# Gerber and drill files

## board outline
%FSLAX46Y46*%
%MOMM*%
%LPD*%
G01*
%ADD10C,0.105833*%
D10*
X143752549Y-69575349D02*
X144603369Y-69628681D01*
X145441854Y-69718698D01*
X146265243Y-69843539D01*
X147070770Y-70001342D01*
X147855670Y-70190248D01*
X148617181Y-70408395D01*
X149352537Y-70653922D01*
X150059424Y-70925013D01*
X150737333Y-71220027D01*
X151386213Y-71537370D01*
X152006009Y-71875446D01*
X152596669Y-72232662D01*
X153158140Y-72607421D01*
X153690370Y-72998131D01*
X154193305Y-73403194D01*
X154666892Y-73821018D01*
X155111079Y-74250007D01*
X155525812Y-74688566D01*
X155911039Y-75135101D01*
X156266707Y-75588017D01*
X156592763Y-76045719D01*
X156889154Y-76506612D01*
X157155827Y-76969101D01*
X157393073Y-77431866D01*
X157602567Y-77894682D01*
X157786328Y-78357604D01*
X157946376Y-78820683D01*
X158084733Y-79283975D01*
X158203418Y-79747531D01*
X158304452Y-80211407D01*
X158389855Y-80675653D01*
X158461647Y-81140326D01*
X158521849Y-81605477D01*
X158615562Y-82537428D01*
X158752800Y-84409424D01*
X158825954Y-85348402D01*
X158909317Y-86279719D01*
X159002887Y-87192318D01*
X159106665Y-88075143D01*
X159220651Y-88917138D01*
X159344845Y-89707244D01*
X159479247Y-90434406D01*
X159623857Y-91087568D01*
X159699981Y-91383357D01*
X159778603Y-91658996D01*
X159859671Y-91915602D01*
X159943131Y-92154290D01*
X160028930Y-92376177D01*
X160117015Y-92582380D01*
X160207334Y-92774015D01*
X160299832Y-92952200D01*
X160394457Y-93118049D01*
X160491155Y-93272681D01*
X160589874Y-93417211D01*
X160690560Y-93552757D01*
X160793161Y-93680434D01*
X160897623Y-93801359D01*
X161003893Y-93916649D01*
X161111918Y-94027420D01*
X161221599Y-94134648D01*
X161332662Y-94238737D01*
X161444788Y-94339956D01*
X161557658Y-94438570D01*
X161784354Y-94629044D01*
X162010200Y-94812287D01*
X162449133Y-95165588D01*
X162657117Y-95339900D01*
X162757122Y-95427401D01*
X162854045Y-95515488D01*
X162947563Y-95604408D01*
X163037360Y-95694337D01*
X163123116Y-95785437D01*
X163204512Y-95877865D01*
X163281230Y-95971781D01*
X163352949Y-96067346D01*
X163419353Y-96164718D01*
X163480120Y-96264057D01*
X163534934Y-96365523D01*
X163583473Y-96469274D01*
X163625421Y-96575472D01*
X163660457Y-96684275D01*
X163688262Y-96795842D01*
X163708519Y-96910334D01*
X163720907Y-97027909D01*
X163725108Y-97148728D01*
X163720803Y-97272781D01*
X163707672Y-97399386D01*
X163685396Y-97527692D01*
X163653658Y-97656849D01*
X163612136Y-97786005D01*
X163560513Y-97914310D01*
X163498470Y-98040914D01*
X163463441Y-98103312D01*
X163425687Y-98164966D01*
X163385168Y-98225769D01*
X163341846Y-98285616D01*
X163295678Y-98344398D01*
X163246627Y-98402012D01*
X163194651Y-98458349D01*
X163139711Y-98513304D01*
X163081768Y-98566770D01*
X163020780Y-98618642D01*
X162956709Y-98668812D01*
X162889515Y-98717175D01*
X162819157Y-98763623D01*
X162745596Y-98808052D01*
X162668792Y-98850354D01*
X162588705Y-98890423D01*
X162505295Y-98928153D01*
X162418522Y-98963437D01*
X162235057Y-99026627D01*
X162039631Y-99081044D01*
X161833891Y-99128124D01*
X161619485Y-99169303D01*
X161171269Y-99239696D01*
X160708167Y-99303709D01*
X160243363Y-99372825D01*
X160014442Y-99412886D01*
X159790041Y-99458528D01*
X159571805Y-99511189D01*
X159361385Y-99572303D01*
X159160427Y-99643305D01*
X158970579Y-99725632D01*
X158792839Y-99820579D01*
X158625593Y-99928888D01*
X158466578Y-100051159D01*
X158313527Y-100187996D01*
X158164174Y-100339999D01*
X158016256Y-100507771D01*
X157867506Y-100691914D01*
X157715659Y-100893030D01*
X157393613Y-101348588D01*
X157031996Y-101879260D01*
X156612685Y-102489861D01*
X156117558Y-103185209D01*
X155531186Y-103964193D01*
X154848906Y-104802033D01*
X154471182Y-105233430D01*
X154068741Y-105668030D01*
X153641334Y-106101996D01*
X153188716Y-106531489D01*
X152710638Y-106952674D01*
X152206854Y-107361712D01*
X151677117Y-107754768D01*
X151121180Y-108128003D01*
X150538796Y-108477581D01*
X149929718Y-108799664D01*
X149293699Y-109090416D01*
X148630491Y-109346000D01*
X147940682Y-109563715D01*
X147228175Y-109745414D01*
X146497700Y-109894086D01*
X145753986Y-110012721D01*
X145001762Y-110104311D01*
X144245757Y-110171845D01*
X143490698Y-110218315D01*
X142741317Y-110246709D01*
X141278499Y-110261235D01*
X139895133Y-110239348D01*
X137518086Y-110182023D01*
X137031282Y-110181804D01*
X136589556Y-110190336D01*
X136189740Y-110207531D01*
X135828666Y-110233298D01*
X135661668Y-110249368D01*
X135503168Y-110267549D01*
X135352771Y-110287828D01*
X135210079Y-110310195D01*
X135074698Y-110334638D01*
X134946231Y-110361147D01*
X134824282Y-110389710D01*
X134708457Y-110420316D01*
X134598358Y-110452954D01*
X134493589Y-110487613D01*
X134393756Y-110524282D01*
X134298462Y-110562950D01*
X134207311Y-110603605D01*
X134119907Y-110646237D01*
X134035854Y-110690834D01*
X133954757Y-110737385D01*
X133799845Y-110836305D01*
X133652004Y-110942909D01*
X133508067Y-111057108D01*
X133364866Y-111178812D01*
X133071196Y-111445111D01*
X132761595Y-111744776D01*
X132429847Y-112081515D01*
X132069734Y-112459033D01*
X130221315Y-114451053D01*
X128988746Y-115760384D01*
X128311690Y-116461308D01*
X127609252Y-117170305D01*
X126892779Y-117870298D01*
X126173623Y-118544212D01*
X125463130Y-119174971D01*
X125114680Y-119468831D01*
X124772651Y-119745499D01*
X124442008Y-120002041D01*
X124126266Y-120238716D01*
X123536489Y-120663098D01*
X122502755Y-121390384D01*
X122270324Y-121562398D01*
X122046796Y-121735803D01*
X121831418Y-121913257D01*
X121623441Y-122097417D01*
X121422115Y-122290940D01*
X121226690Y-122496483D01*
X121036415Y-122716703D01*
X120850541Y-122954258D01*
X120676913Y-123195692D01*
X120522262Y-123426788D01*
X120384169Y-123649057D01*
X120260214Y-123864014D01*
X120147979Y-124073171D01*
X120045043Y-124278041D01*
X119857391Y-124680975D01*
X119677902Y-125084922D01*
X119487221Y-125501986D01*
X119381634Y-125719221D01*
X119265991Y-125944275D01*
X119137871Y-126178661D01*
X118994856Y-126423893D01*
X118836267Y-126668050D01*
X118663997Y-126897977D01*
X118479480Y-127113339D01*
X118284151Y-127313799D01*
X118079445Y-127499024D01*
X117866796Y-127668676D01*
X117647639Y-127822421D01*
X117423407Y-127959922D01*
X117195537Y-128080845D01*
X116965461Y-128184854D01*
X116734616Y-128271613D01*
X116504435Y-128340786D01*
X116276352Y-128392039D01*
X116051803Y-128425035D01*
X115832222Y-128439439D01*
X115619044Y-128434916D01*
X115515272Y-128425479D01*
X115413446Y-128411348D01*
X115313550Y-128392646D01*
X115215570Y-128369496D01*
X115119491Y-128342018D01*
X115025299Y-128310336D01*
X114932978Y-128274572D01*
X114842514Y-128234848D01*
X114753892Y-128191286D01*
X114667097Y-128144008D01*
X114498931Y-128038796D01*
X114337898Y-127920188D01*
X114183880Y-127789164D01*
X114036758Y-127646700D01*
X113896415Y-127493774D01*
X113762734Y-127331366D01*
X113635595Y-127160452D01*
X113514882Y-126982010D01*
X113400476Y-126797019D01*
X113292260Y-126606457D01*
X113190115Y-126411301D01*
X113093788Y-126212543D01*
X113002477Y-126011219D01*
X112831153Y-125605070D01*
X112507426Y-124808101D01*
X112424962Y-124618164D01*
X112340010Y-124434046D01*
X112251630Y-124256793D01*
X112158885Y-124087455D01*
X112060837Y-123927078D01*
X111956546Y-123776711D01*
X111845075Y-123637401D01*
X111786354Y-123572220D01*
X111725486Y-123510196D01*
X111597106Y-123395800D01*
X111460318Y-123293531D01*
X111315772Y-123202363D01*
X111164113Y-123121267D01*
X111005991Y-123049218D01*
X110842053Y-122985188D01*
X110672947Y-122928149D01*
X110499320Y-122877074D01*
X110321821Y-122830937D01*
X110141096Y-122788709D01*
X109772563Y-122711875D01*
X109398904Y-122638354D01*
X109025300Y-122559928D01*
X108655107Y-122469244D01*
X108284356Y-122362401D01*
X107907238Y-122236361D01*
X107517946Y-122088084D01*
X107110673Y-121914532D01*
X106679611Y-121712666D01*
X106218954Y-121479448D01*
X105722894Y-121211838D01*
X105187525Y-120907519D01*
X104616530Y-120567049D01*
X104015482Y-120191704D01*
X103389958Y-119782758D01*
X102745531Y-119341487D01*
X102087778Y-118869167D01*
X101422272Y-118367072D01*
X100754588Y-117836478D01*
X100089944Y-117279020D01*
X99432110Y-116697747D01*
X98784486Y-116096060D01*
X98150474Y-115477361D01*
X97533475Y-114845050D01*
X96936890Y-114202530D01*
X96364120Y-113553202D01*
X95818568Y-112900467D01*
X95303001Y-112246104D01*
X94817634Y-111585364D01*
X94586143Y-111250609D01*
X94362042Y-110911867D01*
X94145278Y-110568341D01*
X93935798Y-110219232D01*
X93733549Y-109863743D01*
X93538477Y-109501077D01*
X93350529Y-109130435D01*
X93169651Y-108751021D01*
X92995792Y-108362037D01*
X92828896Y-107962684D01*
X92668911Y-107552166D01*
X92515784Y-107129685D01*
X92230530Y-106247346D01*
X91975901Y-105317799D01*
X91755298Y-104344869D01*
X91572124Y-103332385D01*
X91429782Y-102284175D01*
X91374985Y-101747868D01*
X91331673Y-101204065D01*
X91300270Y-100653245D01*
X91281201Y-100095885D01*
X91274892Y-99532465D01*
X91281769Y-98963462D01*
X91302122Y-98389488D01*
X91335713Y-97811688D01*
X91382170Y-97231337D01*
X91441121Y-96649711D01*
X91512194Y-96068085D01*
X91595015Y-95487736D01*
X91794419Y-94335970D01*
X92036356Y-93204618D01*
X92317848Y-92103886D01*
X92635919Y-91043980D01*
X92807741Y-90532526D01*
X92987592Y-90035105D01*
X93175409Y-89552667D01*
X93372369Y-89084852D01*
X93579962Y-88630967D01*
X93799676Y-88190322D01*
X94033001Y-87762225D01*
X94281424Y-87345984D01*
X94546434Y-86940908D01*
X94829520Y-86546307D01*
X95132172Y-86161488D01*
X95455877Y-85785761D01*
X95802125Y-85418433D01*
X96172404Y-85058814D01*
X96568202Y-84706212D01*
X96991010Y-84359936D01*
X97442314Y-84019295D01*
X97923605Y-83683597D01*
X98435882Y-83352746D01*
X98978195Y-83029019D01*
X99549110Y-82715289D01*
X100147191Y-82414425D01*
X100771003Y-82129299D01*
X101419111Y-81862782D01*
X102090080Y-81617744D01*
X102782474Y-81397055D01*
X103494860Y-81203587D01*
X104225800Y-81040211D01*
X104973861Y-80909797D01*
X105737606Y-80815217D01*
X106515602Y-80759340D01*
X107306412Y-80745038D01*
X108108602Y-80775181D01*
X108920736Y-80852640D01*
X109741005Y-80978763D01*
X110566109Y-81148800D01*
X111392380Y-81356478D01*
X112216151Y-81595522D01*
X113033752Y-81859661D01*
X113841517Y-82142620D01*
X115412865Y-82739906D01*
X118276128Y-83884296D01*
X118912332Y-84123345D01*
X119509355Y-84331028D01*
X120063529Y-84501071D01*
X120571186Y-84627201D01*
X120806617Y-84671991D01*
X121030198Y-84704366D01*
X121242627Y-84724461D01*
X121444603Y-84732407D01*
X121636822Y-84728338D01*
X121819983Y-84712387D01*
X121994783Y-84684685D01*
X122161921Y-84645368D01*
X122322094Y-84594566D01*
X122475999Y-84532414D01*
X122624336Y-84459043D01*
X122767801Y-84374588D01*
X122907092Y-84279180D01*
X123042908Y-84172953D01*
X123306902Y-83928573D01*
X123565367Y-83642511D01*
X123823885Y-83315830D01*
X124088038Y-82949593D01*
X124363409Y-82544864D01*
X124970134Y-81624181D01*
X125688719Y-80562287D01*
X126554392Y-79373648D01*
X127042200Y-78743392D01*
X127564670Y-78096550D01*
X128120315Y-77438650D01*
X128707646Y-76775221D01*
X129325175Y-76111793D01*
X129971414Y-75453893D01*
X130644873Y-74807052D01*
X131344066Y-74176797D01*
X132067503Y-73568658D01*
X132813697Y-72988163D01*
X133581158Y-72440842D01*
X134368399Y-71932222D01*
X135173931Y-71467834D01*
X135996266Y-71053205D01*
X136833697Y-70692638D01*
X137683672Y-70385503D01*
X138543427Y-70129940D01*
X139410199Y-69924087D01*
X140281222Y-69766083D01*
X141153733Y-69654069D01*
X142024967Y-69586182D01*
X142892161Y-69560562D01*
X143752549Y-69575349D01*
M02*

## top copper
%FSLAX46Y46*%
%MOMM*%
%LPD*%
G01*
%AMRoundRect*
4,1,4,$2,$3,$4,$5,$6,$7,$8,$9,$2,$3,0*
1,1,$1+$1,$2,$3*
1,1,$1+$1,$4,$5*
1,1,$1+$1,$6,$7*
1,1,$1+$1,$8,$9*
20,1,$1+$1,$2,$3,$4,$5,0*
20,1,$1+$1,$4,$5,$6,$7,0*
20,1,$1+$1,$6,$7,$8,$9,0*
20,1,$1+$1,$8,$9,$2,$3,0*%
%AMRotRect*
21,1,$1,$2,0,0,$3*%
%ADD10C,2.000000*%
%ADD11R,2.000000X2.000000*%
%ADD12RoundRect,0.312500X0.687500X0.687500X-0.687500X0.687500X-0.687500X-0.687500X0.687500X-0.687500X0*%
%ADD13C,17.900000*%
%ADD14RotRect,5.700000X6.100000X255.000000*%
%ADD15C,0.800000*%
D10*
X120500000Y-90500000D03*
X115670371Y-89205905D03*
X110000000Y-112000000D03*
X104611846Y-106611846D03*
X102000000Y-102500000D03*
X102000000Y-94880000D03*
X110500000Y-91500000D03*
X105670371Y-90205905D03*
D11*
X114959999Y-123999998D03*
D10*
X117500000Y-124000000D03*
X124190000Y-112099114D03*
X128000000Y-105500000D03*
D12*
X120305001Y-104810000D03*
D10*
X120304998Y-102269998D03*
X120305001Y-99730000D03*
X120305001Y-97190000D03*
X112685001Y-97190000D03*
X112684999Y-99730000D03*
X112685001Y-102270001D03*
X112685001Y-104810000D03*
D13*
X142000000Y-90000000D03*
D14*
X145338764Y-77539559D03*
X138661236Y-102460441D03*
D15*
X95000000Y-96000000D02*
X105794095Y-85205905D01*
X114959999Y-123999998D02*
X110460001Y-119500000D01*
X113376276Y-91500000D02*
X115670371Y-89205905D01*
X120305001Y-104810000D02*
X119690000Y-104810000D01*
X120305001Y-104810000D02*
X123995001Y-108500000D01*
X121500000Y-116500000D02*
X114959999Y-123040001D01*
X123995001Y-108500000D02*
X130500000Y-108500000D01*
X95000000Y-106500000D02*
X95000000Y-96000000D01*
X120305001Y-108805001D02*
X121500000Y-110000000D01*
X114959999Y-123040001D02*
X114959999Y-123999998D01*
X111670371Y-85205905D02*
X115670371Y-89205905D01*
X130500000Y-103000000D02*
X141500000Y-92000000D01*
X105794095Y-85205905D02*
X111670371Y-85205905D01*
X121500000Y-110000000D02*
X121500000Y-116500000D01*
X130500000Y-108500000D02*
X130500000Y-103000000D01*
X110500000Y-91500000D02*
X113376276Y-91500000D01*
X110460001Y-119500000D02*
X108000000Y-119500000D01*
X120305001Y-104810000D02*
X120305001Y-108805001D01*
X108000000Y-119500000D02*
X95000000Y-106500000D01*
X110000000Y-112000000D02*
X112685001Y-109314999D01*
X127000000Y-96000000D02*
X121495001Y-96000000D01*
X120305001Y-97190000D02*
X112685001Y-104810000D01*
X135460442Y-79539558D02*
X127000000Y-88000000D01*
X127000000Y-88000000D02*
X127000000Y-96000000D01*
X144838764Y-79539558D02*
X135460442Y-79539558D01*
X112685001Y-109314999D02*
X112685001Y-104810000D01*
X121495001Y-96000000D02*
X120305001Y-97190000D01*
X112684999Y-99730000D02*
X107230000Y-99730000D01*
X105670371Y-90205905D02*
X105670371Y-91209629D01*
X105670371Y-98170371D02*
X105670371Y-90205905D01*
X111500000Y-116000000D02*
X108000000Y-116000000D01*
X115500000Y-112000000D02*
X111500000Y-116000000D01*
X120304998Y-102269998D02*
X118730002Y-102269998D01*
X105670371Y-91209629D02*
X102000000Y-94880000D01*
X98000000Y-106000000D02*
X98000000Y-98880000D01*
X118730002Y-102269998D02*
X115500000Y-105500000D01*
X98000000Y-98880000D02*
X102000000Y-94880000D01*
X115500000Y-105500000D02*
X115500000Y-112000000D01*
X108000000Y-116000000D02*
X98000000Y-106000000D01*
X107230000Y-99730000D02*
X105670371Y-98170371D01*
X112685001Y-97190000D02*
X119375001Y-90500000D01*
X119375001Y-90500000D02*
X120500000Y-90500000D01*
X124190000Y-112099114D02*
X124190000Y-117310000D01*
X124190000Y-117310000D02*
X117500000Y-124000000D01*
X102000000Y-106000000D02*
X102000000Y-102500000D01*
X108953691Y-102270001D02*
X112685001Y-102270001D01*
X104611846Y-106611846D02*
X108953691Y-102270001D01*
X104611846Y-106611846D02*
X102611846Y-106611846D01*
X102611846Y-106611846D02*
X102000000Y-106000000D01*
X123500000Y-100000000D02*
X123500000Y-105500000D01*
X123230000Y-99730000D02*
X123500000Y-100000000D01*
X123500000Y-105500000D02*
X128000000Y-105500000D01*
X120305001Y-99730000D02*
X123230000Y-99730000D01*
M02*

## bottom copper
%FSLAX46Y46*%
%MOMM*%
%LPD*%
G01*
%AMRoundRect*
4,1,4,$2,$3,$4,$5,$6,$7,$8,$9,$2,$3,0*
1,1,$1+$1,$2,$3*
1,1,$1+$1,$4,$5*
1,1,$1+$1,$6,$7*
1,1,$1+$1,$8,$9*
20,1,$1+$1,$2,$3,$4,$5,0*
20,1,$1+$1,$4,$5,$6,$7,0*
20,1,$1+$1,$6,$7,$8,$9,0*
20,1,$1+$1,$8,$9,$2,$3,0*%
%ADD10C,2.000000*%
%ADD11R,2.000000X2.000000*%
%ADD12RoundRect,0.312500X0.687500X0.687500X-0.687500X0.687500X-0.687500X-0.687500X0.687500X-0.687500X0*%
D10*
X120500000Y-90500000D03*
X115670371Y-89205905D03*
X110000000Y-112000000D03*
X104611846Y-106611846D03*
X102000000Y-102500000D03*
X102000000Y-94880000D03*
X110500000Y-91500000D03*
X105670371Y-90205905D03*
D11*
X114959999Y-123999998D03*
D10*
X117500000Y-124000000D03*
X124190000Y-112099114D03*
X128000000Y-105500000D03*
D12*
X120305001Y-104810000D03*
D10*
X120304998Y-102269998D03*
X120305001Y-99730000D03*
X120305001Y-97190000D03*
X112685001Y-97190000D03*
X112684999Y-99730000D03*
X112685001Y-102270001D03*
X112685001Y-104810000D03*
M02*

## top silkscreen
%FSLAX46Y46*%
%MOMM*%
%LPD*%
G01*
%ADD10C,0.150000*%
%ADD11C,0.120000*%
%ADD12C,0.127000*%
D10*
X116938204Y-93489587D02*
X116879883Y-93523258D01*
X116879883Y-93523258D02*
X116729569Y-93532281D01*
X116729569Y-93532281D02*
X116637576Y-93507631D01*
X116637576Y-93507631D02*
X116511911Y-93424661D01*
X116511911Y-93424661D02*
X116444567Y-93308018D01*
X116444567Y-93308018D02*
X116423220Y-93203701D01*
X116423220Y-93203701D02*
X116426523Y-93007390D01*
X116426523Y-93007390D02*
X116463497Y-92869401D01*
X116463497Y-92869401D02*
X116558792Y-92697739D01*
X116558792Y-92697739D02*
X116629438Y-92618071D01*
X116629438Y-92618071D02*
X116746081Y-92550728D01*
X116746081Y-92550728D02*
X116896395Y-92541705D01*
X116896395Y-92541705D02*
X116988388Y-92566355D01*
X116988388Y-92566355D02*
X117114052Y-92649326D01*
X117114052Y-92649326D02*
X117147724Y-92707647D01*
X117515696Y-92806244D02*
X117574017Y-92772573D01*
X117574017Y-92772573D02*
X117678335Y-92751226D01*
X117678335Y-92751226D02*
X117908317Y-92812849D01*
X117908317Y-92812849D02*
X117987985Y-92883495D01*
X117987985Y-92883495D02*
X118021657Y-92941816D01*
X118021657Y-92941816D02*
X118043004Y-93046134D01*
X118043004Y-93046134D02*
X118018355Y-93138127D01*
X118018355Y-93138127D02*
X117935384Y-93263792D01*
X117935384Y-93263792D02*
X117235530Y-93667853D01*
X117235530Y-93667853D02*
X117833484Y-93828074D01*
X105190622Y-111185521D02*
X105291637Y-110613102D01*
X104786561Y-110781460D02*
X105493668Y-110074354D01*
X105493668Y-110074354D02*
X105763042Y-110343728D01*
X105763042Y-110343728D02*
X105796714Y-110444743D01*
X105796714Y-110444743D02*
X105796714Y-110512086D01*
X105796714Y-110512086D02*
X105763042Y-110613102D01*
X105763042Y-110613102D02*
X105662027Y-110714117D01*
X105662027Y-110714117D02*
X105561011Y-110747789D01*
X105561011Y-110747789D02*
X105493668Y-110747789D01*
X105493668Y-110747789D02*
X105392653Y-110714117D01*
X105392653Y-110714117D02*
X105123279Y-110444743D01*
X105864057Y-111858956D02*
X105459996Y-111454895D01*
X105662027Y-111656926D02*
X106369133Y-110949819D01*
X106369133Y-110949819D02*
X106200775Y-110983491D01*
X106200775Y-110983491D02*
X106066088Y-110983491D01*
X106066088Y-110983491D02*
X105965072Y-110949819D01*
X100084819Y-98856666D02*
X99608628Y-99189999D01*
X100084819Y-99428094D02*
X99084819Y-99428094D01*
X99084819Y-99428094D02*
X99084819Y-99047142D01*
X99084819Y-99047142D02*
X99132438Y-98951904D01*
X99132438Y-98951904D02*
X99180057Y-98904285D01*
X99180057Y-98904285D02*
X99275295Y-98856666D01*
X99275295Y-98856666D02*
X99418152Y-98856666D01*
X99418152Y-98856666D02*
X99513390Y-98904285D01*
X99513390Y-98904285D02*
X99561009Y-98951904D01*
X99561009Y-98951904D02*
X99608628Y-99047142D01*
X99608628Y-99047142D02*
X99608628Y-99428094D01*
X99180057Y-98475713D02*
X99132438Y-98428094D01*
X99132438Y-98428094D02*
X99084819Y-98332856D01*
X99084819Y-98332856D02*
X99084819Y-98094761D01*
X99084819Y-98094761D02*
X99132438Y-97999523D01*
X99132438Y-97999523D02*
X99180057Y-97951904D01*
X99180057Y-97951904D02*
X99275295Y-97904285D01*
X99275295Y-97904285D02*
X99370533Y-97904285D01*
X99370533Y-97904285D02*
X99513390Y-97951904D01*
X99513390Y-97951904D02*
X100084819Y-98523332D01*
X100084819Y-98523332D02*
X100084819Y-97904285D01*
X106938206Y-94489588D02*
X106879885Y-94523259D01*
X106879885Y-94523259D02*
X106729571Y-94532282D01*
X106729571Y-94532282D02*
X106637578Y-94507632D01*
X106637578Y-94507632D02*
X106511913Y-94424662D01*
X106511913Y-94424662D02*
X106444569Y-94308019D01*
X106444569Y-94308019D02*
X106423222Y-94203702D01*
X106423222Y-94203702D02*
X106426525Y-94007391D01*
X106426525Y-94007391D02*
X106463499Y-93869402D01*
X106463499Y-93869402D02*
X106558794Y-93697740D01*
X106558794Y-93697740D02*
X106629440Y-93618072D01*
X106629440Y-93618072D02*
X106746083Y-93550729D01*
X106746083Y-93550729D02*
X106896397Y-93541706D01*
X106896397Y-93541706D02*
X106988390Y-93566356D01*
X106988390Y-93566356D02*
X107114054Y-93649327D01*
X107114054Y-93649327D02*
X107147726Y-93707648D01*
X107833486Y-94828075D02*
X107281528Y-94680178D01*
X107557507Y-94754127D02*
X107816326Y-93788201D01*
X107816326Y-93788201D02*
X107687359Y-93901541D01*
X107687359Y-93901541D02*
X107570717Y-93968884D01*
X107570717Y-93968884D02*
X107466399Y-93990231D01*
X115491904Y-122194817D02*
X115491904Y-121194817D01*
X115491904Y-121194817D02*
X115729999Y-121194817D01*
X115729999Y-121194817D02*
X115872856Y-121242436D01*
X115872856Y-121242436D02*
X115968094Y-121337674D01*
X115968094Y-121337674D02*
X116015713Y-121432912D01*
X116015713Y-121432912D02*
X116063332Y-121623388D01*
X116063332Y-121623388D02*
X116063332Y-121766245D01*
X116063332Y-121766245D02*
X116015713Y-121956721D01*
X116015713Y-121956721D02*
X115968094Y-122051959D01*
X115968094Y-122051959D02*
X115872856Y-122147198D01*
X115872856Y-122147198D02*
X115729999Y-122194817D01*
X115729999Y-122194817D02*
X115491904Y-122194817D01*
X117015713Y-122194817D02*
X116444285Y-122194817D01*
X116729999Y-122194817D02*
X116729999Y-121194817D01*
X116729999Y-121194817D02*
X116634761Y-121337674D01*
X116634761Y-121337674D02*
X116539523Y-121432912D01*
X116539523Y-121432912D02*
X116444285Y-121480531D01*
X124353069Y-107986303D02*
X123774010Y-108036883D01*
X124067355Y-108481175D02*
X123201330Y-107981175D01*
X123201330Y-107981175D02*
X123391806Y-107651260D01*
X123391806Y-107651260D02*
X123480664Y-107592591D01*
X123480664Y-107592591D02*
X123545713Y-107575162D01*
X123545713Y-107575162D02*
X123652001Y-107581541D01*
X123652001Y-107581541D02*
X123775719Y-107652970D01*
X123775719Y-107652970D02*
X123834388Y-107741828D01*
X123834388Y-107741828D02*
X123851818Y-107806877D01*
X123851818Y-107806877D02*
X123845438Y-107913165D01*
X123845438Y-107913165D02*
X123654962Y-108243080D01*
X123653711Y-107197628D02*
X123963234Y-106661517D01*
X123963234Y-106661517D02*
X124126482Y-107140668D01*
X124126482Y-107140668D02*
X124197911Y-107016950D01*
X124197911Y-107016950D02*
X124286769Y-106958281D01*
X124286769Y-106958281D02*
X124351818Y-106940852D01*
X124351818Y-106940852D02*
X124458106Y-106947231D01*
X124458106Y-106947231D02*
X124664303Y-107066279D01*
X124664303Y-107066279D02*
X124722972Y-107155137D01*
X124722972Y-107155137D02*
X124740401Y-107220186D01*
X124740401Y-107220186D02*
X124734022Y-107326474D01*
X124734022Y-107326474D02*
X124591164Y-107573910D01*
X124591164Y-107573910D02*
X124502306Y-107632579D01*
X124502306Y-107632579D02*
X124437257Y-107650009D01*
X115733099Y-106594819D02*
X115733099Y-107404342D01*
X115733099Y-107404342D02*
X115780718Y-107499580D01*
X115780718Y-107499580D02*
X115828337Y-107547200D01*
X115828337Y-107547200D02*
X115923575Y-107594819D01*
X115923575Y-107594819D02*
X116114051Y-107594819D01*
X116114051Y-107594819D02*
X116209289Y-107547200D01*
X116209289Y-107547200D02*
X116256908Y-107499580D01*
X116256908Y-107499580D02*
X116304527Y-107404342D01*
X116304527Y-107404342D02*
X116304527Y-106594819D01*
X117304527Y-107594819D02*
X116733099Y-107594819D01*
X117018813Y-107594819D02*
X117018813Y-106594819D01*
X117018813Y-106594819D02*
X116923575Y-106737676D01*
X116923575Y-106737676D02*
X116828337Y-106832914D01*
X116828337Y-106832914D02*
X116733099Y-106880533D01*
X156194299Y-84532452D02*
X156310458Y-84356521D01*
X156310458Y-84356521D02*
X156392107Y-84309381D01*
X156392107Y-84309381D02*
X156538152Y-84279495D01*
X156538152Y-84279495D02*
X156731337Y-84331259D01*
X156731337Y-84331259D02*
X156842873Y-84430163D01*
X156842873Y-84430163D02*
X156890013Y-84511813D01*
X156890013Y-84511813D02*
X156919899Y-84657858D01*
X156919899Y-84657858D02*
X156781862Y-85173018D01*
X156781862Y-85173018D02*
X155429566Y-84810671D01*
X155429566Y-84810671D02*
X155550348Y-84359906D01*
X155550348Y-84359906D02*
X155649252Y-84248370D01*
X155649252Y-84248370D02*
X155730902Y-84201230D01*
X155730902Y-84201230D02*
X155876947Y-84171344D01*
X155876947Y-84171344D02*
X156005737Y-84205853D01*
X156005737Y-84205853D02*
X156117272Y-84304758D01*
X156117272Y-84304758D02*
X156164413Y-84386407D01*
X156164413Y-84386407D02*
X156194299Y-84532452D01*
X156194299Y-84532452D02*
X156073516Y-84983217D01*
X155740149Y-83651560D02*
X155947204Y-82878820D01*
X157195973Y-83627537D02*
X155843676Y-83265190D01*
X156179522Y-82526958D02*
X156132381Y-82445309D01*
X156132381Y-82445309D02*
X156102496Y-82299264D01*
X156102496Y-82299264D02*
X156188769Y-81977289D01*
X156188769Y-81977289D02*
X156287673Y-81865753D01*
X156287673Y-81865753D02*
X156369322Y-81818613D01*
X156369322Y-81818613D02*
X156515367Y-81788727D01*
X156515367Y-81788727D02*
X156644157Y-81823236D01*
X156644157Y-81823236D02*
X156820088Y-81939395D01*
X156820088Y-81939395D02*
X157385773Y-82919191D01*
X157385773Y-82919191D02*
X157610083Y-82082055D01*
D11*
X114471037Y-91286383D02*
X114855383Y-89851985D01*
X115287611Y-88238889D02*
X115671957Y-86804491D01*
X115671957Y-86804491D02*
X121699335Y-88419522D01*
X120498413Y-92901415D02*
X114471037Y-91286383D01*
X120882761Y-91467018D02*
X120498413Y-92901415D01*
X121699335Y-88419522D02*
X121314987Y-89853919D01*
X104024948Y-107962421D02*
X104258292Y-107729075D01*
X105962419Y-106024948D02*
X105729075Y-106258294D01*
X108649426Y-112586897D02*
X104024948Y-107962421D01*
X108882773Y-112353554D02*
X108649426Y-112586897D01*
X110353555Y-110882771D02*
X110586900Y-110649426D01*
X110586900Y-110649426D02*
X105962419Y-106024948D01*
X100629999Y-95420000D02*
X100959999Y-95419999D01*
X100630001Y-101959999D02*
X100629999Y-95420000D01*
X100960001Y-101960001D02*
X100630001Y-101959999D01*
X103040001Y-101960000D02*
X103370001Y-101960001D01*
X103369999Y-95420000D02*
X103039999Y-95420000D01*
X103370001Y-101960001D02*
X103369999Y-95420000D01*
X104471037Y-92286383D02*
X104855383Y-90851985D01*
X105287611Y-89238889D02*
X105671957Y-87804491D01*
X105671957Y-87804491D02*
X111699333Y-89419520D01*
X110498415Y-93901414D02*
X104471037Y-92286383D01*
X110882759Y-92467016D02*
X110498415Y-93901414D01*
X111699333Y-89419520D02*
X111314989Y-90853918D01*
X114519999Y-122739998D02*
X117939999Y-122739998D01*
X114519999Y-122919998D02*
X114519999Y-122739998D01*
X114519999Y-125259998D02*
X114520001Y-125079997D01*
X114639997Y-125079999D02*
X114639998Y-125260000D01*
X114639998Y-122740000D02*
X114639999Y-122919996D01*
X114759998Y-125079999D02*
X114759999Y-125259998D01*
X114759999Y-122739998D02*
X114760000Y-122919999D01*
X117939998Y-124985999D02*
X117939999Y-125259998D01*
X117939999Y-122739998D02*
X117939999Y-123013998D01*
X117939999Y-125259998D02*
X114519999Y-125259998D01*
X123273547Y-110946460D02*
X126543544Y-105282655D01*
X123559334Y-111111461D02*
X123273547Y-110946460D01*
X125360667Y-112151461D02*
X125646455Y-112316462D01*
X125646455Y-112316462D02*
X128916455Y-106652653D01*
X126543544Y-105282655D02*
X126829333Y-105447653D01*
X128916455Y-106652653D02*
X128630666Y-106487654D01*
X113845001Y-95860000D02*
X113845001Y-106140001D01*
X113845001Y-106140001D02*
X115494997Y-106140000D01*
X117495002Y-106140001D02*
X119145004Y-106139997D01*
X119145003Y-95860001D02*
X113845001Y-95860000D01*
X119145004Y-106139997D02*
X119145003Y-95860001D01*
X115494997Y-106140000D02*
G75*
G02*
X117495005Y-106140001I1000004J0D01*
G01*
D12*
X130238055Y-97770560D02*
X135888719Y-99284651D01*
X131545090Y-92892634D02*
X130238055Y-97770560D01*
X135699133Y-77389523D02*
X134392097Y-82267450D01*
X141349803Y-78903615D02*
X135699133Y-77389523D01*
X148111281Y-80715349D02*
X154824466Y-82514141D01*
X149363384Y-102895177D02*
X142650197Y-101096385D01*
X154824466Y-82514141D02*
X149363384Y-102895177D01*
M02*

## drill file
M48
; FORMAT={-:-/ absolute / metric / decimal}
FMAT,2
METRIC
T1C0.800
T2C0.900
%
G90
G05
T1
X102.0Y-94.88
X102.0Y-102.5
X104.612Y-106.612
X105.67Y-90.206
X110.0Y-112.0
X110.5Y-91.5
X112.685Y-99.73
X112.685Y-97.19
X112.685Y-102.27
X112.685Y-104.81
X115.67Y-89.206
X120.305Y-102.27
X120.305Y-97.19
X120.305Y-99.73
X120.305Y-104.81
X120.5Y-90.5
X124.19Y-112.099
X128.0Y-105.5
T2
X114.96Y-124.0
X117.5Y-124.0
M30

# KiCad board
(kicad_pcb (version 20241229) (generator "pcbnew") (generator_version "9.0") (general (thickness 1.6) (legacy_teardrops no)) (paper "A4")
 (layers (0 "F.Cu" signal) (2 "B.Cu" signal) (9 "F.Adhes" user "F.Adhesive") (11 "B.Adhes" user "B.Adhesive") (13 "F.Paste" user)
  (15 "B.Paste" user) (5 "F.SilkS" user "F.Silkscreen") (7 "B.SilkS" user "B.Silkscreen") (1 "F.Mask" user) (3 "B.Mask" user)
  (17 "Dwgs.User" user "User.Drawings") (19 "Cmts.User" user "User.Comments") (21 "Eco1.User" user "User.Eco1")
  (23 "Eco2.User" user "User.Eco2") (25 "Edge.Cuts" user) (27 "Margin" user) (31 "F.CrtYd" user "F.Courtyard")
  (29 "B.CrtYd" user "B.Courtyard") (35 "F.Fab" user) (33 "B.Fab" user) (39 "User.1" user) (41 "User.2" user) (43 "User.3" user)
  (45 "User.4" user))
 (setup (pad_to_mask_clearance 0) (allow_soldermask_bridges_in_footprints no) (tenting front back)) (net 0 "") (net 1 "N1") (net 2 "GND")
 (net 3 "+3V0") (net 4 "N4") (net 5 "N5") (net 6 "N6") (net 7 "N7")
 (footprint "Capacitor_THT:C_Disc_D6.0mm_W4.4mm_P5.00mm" (layer "F.Cu") (at 120.5 90.5 165)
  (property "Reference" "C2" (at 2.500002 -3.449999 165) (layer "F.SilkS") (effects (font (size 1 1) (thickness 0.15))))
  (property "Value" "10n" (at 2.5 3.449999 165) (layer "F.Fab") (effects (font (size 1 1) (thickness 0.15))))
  (fp_line (start 5.62 -2.319998) (end 5.62 -0.835) (stroke (width 0.12) (type solid)) (layer "F.SilkS"))
  (fp_line (start 5.62 0.835) (end 5.62 2.319998) (stroke (width 0.12) (type solid)) (layer "F.SilkS"))
  (fp_line (start 5.62 2.319998) (end -0.620001 2.319998) (stroke (width 0.12) (type solid)) (layer "F.SilkS"))
  (fp_line (start -0.619999 -2.32) (end 5.62 -2.319998) (stroke (width 0.12) (type solid)) (layer "F.SilkS"))
  (fp_line (start -0.620001 -0.835002) (end -0.619999 -2.32) (stroke (width 0.12) (type solid)) (layer "F.SilkS"))
  (fp_line (start -0.620001 2.319998) (end -0.619999 0.835) (stroke (width 0.12) (type solid)) (layer "F.SilkS"))
  (pad "1" thru_hole circle (at 0 0 165) (size 2 2) (drill 0.8) (layers "*.Cu" "*.Mask") (remove_unused_layers no) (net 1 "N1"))
  (pad "2" thru_hole circle (at 5 0 165) (size 2 2) (drill 0.8) (layers "*.Cu" "*.Mask") (remove_unused_layers no) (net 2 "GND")))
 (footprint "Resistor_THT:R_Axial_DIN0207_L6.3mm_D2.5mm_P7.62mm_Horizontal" (layer "F.Cu") (at 110 112 135)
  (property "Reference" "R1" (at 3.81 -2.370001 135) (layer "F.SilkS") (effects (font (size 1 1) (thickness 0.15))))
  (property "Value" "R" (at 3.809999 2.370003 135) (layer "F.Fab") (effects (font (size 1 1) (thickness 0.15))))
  (fp_line (start 7.079999 -1.37) (end 7.080001 -1.040001) (stroke (width 0.12) (type solid)) (layer "F.SilkS"))
  (fp_line (start 7.080001 1.369999) (end 7.079999 1.039999) (stroke (width 0.12) (type solid)) (layer "F.SilkS"))
  (fp_line (start 0.540001 -1.369999) (end 7.079999 -1.37) (stroke (width 0.12) (type solid)) (layer "F.SilkS"))
  (fp_line (start 0.539998 -1.039999) (end 0.540001 -1.369999) (stroke (width 0.12) (type solid)) (layer "F.SilkS"))
  (fp_line (start 0.539999 1.040001) (end 0.539999 1.370001) (stroke (width 0.12) (type solid)) (layer "F.SilkS"))
  (fp_line (start 0.539999 1.370001) (end 7.080001 1.369999) (stroke (width 0.12) (type solid)) (layer "F.SilkS"))
  (pad "1" thru_hole circle (at 0 0 135) (size 2 2) (drill 0.8) (layers "*.Cu" "*.Mask") (remove_unused_layers no) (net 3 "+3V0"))
  (pad "2" thru_hole circle (at 7.62 0 135) (size 2 2) (drill 0.8) (layers "*.Cu" "*.Mask") (remove_unused_layers no) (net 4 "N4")))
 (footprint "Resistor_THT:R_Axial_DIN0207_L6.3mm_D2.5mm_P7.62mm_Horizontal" (layer "F.Cu") (at 102 102.5 90)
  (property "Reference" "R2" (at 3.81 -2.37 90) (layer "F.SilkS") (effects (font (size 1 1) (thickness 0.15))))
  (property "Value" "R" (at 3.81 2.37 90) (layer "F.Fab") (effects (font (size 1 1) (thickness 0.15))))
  (fp_line (start 7.08 -1.370001) (end 7.080001 -1.040001) (stroke (width 0.12) (type solid)) (layer "F.SilkS"))
  (fp_line (start 0.540001 -1.369999) (end 7.08 -1.370001) (stroke (width 0.12) (type solid)) (layer "F.SilkS"))
  (fp_line (start 0.539999 -1.039999) (end 0.540001 -1.369999) (stroke (width 0.12) (type solid)) (layer "F.SilkS"))
  (fp_line (start 0.54 1.040001) (end 0.539999 1.370001) (stroke (width 0.12) (type solid)) (layer "F.SilkS"))
  (fp_line (start 7.08 1.369999) (end 7.08 1.039999) (stroke (width 0.12) (type solid)) (layer "F.SilkS"))
  (fp_line (start 0.539999 1.370001) (end 7.08 1.369999) (stroke (width 0.12) (type solid)) (layer "F.SilkS"))
  (pad "1" thru_hole circle (at 0 0 90) (size 2 2) (drill 0.8) (layers "*.Cu" "*.Mask") (remove_unused_layers no) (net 4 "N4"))
  (pad "2" thru_hole circle (at 7.62 0 90) (size 2 2) (drill 0.8) (layers "*.Cu" "*.Mask") (remove_unused_layers no) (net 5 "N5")))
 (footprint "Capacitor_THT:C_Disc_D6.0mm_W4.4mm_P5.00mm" (layer "F.Cu") (at 110.5 91.5 165)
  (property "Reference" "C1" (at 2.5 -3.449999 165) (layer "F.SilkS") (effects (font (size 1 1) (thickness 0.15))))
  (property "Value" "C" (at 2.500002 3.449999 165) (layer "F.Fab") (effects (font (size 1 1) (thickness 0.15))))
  (fp_line (start 5.62 -2.319998) (end 5.62 -0.835) (stroke (width 0.12) (type solid)) (layer "F.SilkS"))
  (fp_line (start 5.62 0.835) (end 5.62 2.319998) (stroke (width 0.12) (type solid)) (layer "F.SilkS"))
  (fp_line (start 5.62 2.319998) (end -0.619999 2.32) (stroke (width 0.12) (type solid)) (layer "F.SilkS"))
  (fp_line (start -0.620001 -2.319998) (end 5.62 -2.319998) (stroke (width 0.12) (type solid)) (layer "F.SilkS"))
  (fp_line (start -0.619999 -0.835) (end -0.620001 -2.319998) (stroke (width 0.12) (type solid)) (layer "F.SilkS"))
  (fp_line (start -0.619999 2.32) (end -0.620001 0.835002) (stroke (width 0.12) (type solid)) (layer "F.SilkS"))
  (pad "1" thru_hole circle (at 0 0 165) (size 2 2) (drill 0.8) (layers "*.Cu" "*.Mask") (remove_unused_layers no) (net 2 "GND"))
  (pad "2" thru_hole circle (at 5 0 165) (size 2 2) (drill 0.8) (layers "*.Cu" "*.Mask") (remove_unused_layers no) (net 5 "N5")))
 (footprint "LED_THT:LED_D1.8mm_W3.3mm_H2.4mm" (layer "F.Cu") (at 114.959999 123.999998)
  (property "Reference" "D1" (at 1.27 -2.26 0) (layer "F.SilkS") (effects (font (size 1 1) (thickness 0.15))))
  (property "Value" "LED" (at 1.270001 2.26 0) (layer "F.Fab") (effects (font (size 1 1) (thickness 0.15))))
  (fp_line (start -0.44 -1.26) (end 2.98 -1.26) (stroke (width 0.12) (type solid)) (layer "F.SilkS"))
  (fp_line (start -0.44 -1.08) (end -0.44 -1.26) (stroke (width 0.12) (type solid)) (layer "F.SilkS"))
  (fp_line (start -0.44 1.26) (end -0.439998 1.079999) (stroke (width 0.12) (type solid)) (layer "F.SilkS"))
  (fp_line (start -0.320002 1.080001) (end -0.320001 1.260002) (stroke (width 0.12) (type solid)) (layer "F.SilkS"))
  (fp_line (start -0.320001 -1.259998) (end -0.32 -1.080002) (stroke (width 0.12) (type solid)) (layer "F.SilkS"))
  (fp_line (start -0.200001 1.080001) (end -0.2 1.26) (stroke (width 0.12) (type solid)) (layer "F.SilkS"))
  (fp_line (start -0.2 -1.26) (end -0.199999 -1.079999) (stroke (width 0.12) (type solid)) (layer "F.SilkS"))
  (fp_line (start 2.979999 0.986001) (end 2.98 1.26) (stroke (width 0.12) (type solid)) (layer "F.SilkS"))
  (fp_line (start 2.98 -1.26) (end 2.98 -0.986) (stroke (width 0.12) (type solid)) (layer "F.SilkS"))
  (fp_line (start 2.98 1.26) (end -0.44 1.26) (stroke (width 0.12) (type solid)) (layer "F.SilkS"))
  (pad "1" thru_hole rect (at 0 0) (size 2 2) (drill 0.9) (layers "*.Cu" "*.Mask") (remove_unused_layers no) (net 2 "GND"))
  (pad "2" thru_hole circle (at 2.540001 0.000002) (size 2 2) (drill 0.9) (layers "*.Cu" "*.Mask") (remove_unused_layers no) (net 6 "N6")))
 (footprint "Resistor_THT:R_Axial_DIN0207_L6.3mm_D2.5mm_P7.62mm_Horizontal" (layer "F.Cu") (at 124.19 112.099114 60)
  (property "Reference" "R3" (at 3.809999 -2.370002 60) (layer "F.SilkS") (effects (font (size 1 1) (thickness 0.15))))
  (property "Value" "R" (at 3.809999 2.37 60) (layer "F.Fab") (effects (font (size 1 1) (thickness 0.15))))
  (fp_line (start 0.540001 -1.369999) (end 7.079999 -1.370001) (stroke (width 0.12) (type solid)) (layer "F.SilkS"))
  (fp_line (start 0.54 -1.039999) (end 0.540001 -1.369999) (stroke (width 0.12) (type solid)) (layer "F.SilkS"))
  (fp_line (start 0.54 1.040001) (end 0.539999 1.370001) (stroke (width 0.12) (type solid)) (layer "F.SilkS"))
  (fp_line (start 0.539999 1.370001) (end 7.080001 1.37) (stroke (width 0.12) (type solid)) (layer "F.SilkS"))
  (fp_line (start 7.079999 -1.370001) (end 7.080001 -1.040001) (stroke (width 0.12) (type solid)) (layer "F.SilkS"))
  (fp_line (start 7.080001 1.37) (end 7.08 1.04) (stroke (width 0.12) (type solid)) (layer "F.SilkS"))
  (pad "1" thru_hole circle (at 0 0 60) (size 2 2) (drill 0.8) (layers "*.Cu" "*.Mask") (remove_unused_layers no) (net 6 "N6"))
  (pad "2" thru_hole circle (at 7.62 0 60) (size 2 2) (drill 0.8) (layers "*.Cu" "*.Mask") (remove_unused_layers no) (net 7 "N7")))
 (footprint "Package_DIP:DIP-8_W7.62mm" (layer "F.Cu") (at 120.305001 104.81 180)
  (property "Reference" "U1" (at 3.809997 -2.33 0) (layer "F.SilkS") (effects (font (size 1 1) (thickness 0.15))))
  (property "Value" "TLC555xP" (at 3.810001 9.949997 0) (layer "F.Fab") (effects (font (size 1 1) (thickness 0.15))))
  (fp_line (start 6.46 8.95) (end 6.46 -1.330001) (stroke (width 0.12) (type solid)) (layer "F.SilkS"))
  (fp_line (start 6.46 -1.330001) (end 4.810004 -1.33) (stroke (width 0.12) (type solid)) (layer "F.SilkS"))
  (fp_line (start 2.809999 -1.330001) (end 1.159997 -1.329997) (stroke (width 0.12) (type solid)) (layer "F.SilkS"))
  (fp_line (start 1.159998 8.949999) (end 6.46 8.95) (stroke (width 0.12) (type solid)) (layer "F.SilkS"))
  (fp_line (start 1.159997 -1.329997) (end 1.159998 8.949999) (stroke (width 0.12) (type solid)) (layer "F.SilkS"))
  (fp_arc (start 4.810004 -1.33) (mid 3.81 -0.33) (end 2.809999 -1.330001) (stroke (width 0.12) (type solid)) (layer "F.SilkS"))
  (pad "1" thru_hole roundrect (at 0 0 180) (size 2 2) (drill 0.8) (layers "*.Cu" "*.Mask") (remove_unused_layers no)
   (roundrect_rratio 0.15625) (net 2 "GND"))
  (pad "2" thru_hole circle (at 0.000003 2.540002 180) (size 2 2) (drill 0.8) (layers "*.Cu" "*.Mask") (remove_unused_layers no)
   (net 5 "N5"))
  (pad "3" thru_hole circle (at 0 5.08 180) (size 2 2) (drill 0.8) (layers "*.Cu" "*.Mask") (remove_unused_layers no) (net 7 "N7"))
  (pad "4" thru_hole circle (at 0 7.62 180) (size 2 2) (drill 0.8) (layers "*.Cu" "*.Mask") (remove_unused_layers no) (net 3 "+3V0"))
  (pad "5" thru_hole circle (at 7.62 7.62 180) (size 2 2) (drill 0.8) (layers "*.Cu" "*.Mask") (remove_unused_layers no) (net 1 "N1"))
  (pad "6" thru_hole circle (at 7.620002 5.08 180) (size 2 2) (drill 0.8) (layers "*.Cu" "*.Mask") (remove_unused_layers no) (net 5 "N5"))
  (pad "7" thru_hole circle (at 7.62 2.539999 180) (size 2 2) (drill 0.8) (layers "*.Cu" "*.Mask") (remove_unused_layers no) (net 4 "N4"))
  (pad "8" thru_hole circle (at 7.62 0 180) (size 2 2) (drill 0.8) (layers "*.Cu" "*.Mask") (remove_unused_layers no) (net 3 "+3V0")))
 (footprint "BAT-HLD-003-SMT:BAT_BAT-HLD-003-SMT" (layer "F.Cu") (at 142 90 -105)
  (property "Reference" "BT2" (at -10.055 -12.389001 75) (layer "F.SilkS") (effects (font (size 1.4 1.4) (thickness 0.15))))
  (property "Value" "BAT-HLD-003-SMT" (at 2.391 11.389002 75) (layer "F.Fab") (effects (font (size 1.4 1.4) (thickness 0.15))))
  (fp_line (start 10.55 9.349998) (end 10.55 3.5) (stroke (width 0.127) (type solid)) (layer "F.SilkS"))
  (fp_line (start 5.5 9.349999) (end 10.55 9.349998) (stroke (width 0.127) (type solid)) (layer "F.SilkS"))
  (fp_line (start -10.550001 9.350002) (end -5.5 9.350001) (stroke (width 0.127) (type solid)) (layer "F.SilkS"))
  (fp_line (start -10.550001 3.499998) (end -10.550001 9.350002) (stroke (width 0.127) (type solid)) (layer "F.SilkS"))
  (fp_line (start -10.55 -3.5) (end -10.550001 -10.45) (stroke (width 0.127) (type solid)) (layer "F.SilkS"))
  (fp_line (start 10.550001 -10.45) (end 10.550001 -3.499998) (stroke (width 0.127) (type solid)) (layer "F.SilkS"))
  (fp_line (start -10.550001 -10.45) (end 10.550001 -10.45) (stroke (width 0.127) (type solid)) (layer "F.SilkS"))
  (pad "N" smd circle (at 0 0 255) (size 17.9 17.9) (layers "F.Cu" "F.Mask") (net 2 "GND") (solder_mask_margin 0.102))
  (pad "P1" smd rect (at -12.899998 0.000001 255) (size 5.7 6.1) (layers "F.Cu" "F.Mask" "F.Paste") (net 3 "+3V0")
   (solder_mask_margin 0.102))
  (pad "P2" smd rect (at 12.899998 -0.000001 255) (size 5.7 6.1) (layers "F.Cu" "F.Mask" "F.Paste") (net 3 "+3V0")
   (solder_mask_margin 0.102)))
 (gr_poly
  (pts (xy 143.752549 69.575349) (xy 144.603369 69.628681) (xy 145.441854 69.718698) (xy 146.265243 69.843539) (xy 147.07077 70.001342)
   (xy 147.85567 70.190248) (xy 148.617181 70.408395) (xy 149.352537 70.653922) (xy 150.059424 70.925013) (xy 150.737333 71.220027)
   (xy 151.386213 71.53737) (xy 152.006009 71.875446) (xy 152.596669 72.232662) (xy 153.15814 72.607421) (xy 153.69037 72.998131)
   (xy 154.193305 73.403194) (xy 154.666892 73.821018) (xy 155.111079 74.250007) (xy 155.525812 74.688566) (xy 155.911039 75.135101)
   (xy 156.266707 75.588017) (xy 156.592763 76.045719) (xy 156.889154 76.506612) (xy 157.155827 76.969101) (xy 157.393073 77.431866)
   (xy 157.602567 77.894682) (xy 157.786328 78.357604) (xy 157.946376 78.820683) (xy 158.084733 79.283975) (xy 158.203418 79.747531)
   (xy 158.304452 80.211407) (xy 158.389855 80.675653) (xy 158.461647 81.140326) (xy 158.521849 81.605477) (xy 158.615562 82.537428)
   (xy 158.7528 84.409424) (xy 158.825954 85.348402) (xy 158.909317 86.279719) (xy 159.002887 87.192318) (xy 159.106665 88.075143)
   (xy 159.220651 88.917138) (xy 159.344845 89.707244) (xy 159.479247 90.434406) (xy 159.623857 91.087568) (xy 159.699981 91.383357)
   (xy 159.778603 91.658996) (xy 159.859671 91.915602) (xy 159.943131 92.15429) (xy 160.02893 92.376177) (xy 160.117015 92.58238)
   (xy 160.207334 92.774015) (xy 160.299832 92.9522) (xy 160.394457 93.118049) (xy 160.491155 93.272681) (xy 160.589874 93.417211)
   (xy 160.69056 93.552757) (xy 160.793161 93.680434) (xy 160.897623 93.801359) (xy 161.003893 93.916649) (xy 161.111918 94.02742)
   (xy 161.221599 94.134648) (xy 161.332662 94.238737) (xy 161.444788 94.339956) (xy 161.557658 94.43857) (xy 161.784354 94.629044)
   (xy 162.0102 94.812287) (xy 162.449133 95.165588) (xy 162.657117 95.3399) (xy 162.757122 95.427401) (xy 162.854045 95.515488)
   (xy 162.947563 95.604408) (xy 163.03736 95.694337) (xy 163.123116 95.785437) (xy 163.204512 95.877865) (xy 163.28123 95.971781)
   (xy 163.352949 96.067346) (xy 163.419353 96.164718) (xy 163.48012 96.264057) (xy 163.534934 96.365523) (xy 163.583473 96.469274)
   (xy 163.625421 96.575472) (xy 163.660457 96.684275) (xy 163.688262 96.795842) (xy 163.708519 96.910334) (xy 163.720907 97.027909)
   (xy 163.725108 97.148728) (xy 163.720803 97.272781) (xy 163.707672 97.399386) (xy 163.685396 97.527692) (xy 163.653658 97.656849)
   (xy 163.612136 97.786005) (xy 163.560513 97.91431) (xy 163.49847 98.040914) (xy 163.463441 98.103312) (xy 163.425687 98.164966)
   (xy 163.385168 98.225769) (xy 163.341846 98.285616) (xy 163.295678 98.344398) (xy 163.246627 98.402012) (xy 163.194651 98.458349)
   (xy 163.139711 98.513304) (xy 163.081768 98.56677) (xy 163.02078 98.618642) (xy 162.956709 98.668812) (xy 162.889515 98.717175)
   (xy 162.819157 98.763623) (xy 162.745596 98.808052) (xy 162.668792 98.850354) (xy 162.588705 98.890423) (xy 162.505295 98.928153)
   (xy 162.418522 98.963437) (xy 162.235057 99.026627) (xy 162.039631 99.081044) (xy 161.833891 99.128124) (xy 161.619485 99.169303)
   (xy 161.171269 99.239696) (xy 160.708167 99.303709) (xy 160.243363 99.372825) (xy 160.014442 99.412886) (xy 159.790041 99.458528)
   (xy 159.571805 99.511189) (xy 159.361385 99.572303) (xy 159.160427 99.643305) (xy 158.970579 99.725632) (xy 158.792839 99.820579)
   (xy 158.625593 99.928888) (xy 158.466578 100.051159) (xy 158.313527 100.187996) (xy 158.164174 100.339999) (xy 158.016256 100.507771)
   (xy 157.867506 100.691914) (xy 157.715659 100.89303) (xy 157.393613 101.348588) (xy 157.031996 101.87926) (xy 156.612685 102.489861)
   (xy 156.117558 103.185209) (xy 155.531186 103.964193) (xy 154.848906 104.802033) (xy 154.471182 105.23343) (xy 154.068741 105.66803)
   (xy 153.641334 106.101996) (xy 153.188716 106.531489) (xy 152.710638 106.952674) (xy 152.206854 107.361712) (xy 151.677117 107.754768)
   (xy 151.12118 108.128003) (xy 150.538796 108.477581) (xy 149.929718 108.799664) (xy 149.293699 109.090416) (xy 148.630491 109.346)
   (xy 147.940682 109.563715) (xy 147.228175 109.745414) (xy 146.4977 109.894086) (xy 145.753986 110.012721) (xy 145.001762 110.104311)
   (xy 144.245757 110.171845) (xy 143.490698 110.218315) (xy 142.741317 110.246709) (xy 141.278499 110.261235) (xy 139.895133 110.239348)
   (xy 137.518086 110.182023) (xy 137.031282 110.181804) (xy 136.589556 110.190336) (xy 136.18974 110.207531) (xy 135.828666 110.233298)
   (xy 135.661668 110.249368) (xy 135.503168 110.267549) (xy 135.352771 110.287828) (xy 135.210079 110.310195) (xy 135.074698 110.334638)
   (xy 134.946231 110.361147) (xy 134.824282 110.38971) (xy 134.708457 110.420316) (xy 134.598358 110.452954) (xy 134.493589 110.487613)
   (xy 134.393756 110.524282) (xy 134.298462 110.56295) (xy 134.207311 110.603605) (xy 134.119907 110.646237) (xy 134.035854 110.690834)
   (xy 133.954757 110.737385) (xy 133.799845 110.836305) (xy 133.652004 110.942909) (xy 133.508067 111.057108) (xy 133.364866 111.178812)
   (xy 133.071196 111.445111) (xy 132.761595 111.744776) (xy 132.429847 112.081515) (xy 132.069734 112.459033) (xy 130.221315 114.451053)
   (xy 128.988746 115.760384) (xy 128.31169 116.461308) (xy 127.609252 117.170305) (xy 126.892779 117.870298) (xy 126.173623 118.544212)
   (xy 125.46313 119.174971) (xy 125.11468 119.468831) (xy 124.772651 119.745499) (xy 124.442008 120.002041) (xy 124.126266 120.238716)
   (xy 123.536489 120.663098) (xy 122.502755 121.390384) (xy 122.270324 121.562398) (xy 122.046796 121.735803) (xy 121.831418 121.913257)
   (xy 121.623441 122.097417) (xy 121.422115 122.29094) (xy 121.22669 122.496483) (xy 121.036415 122.716703) (xy 120.850541 122.954258)
   (xy 120.676913 123.195692) (xy 120.522262 123.426788) (xy 120.384169 123.649057) (xy 120.260214 123.864014) (xy 120.147979 124.073171)
   (xy 120.045043 124.278041) (xy 119.857391 124.680975) (xy 119.677902 125.084922) (xy 119.487221 125.501986) (xy 119.381634 125.719221)
   (xy 119.265991 125.944275) (xy 119.137871 126.178661) (xy 118.994856 126.423893) (xy 118.836267 126.66805) (xy 118.663997 126.897977)
   (xy 118.47948 127.113339) (xy 118.284151 127.313799) (xy 118.079445 127.499024) (xy 117.866796 127.668676) (xy 117.647639 127.822421)
   (xy 117.423407 127.959922) (xy 117.195537 128.080845) (xy 116.965461 128.184854) (xy 116.734616 128.271613) (xy 116.504435 128.340786)
   (xy 116.276352 128.392039) (xy 116.051803 128.425035) (xy 115.832222 128.439439) (xy 115.619044 128.434916) (xy 115.515272 128.425479)
   (xy 115.413446 128.411348) (xy 115.31355 128.392646) (xy 115.21557 128.369496) (xy 115.119491 128.342018) (xy 115.025299 128.310336)
   (xy 114.932978 128.274572) (xy 114.842514 128.234848) (xy 114.753892 128.191286) (xy 114.667097 128.144008) (xy 114.498931 128.038796)
   (xy 114.337898 127.920188) (xy 114.18388 127.789164) (xy 114.036758 127.6467) (xy 113.896415 127.493774) (xy 113.762734 127.331366)
   (xy 113.635595 127.160452) (xy 113.514882 126.98201) (xy 113.400476 126.797019) (xy 113.29226 126.606457) (xy 113.190115 126.411301)
   (xy 113.093788 126.212543) (xy 113.002477 126.011219) (xy 112.831153 125.60507) (xy 112.507426 124.808101) (xy 112.424962 124.618164)
   (xy 112.34001 124.434046) (xy 112.25163 124.256793) (xy 112.158885 124.087455) (xy 112.060837 123.927078) (xy 111.956546 123.776711)
   (xy 111.845075 123.637401) (xy 111.786354 123.57222) (xy 111.725486 123.510196) (xy 111.597106 123.3958) (xy 111.460318 123.293531)
   (xy 111.315772 123.202363) (xy 111.164113 123.121267) (xy 111.005991 123.049218) (xy 110.842053 122.985188) (xy 110.672947 122.928149)
   (xy 110.49932 122.877074) (xy 110.321821 122.830937) (xy 110.141096 122.788709) (xy 109.772563 122.711875) (xy 109.398904 122.638354)
   (xy 109.0253 122.559928) (xy 108.655107 122.469244) (xy 108.284356 122.362401) (xy 107.907238 122.236361) (xy 107.517946 122.088084)
   (xy 107.110673 121.914532) (xy 106.679611 121.712666) (xy 106.218954 121.479448) (xy 105.722894 121.211838) (xy 105.187525 120.907519)
   (xy 104.61653 120.567049) (xy 104.015482 120.191704) (xy 103.389958 119.782758) (xy 102.745531 119.341487) (xy 102.087778 118.869167)
   (xy 101.422272 118.367072) (xy 100.754588 117.836478) (xy 100.089944 117.27902) (xy 99.43211 116.697747) (xy 98.784486 116.09606)
   (xy 98.150474 115.477361) (xy 97.533475 114.84505) (xy 96.93689 114.20253) (xy 96.36412 113.553202) (xy 95.818568 112.900467)
   (xy 95.303001 112.246104) (xy 94.817634 111.585364) (xy 94.586143 111.250609) (xy 94.362042 110.911867) (xy 94.145278 110.568341)
   (xy 93.935798 110.219232) (xy 93.733549 109.863743) (xy 93.538477 109.501077) (xy 93.350529 109.130435) (xy 93.169651 108.751021)
   (xy 92.995792 108.362037) (xy 92.828896 107.962684) (xy 92.668911 107.552166) (xy 92.515784 107.129685) (xy 92.23053 106.247346)
   (xy 91.975901 105.317799) (xy 91.755298 104.344869) (xy 91.572124 103.332385) (xy 91.429782 102.284175) (xy 91.374985 101.747868)
   (xy 91.331673 101.204065) (xy 91.30027 100.653245) (xy 91.281201 100.095885) (xy 91.274892 99.532465) (xy 91.281769 98.963462)
   (xy 91.302122 98.389488) (xy 91.335713 97.811688) (xy 91.38217 97.231337) (xy 91.441121 96.649711) (xy 91.512194 96.068085)
   (xy 91.595015 95.487736) (xy 91.794419 94.33597) (xy 92.036356 93.204618) (xy 92.317848 92.103886) (xy 92.635919 91.04398)
   (xy 92.807741 90.532526) (xy 92.987592 90.035105) (xy 93.175409 89.552667) (xy 93.372369 89.084852) (xy 93.579962 88.630967)
   (xy 93.799676 88.190322) (xy 94.033001 87.762225) (xy 94.281424 87.345984) (xy 94.546434 86.940908) (xy 94.82952 86.546307)
   (xy 95.132172 86.161488) (xy 95.455877 85.785761) (xy 95.802125 85.418433) (xy 96.172404 85.058814) (xy 96.568202 84.706212)
   (xy 96.99101 84.359936) (xy 97.442314 84.019295) (xy 97.923605 83.683597) (xy 98.435882 83.352746) (xy 98.978195 83.029019)
   (xy 99.54911 82.715289) (xy 100.147191 82.414425) (xy 100.771003 82.129299) (xy 101.419111 81.862782) (xy 102.09008 81.617744)
   (xy 102.782474 81.397055) (xy 103.49486 81.203587) (xy 104.2258 81.040211) (xy 104.973861 80.909797) (xy 105.737606 80.815217)
   (xy 106.515602 80.75934) (xy 107.306412 80.745038) (xy 108.108602 80.775181) (xy 108.920736 80.85264) (xy 109.741005 80.978763)
   (xy 110.566109 81.1488) (xy 111.39238 81.356478) (xy 112.216151 81.595522) (xy 113.033752 81.859661) (xy 113.841517 82.14262)
   (xy 115.412865 82.739906) (xy 118.276128 83.884296) (xy 118.912332 84.123345) (xy 119.509355 84.331028) (xy 120.063529 84.501071)
   (xy 120.571186 84.627201) (xy 120.806617 84.671991) (xy 121.030198 84.704366) (xy 121.242627 84.724461) (xy 121.444603 84.732407)
   (xy 121.636822 84.728338) (xy 121.819983 84.712387) (xy 121.994783 84.684685) (xy 122.161921 84.645368) (xy 122.322094 84.594566)
   (xy 122.475999 84.532414) (xy 122.624336 84.459043) (xy 122.767801 84.374588) (xy 122.907092 84.27918) (xy 123.042908 84.172953)
   (xy 123.306902 83.928573) (xy 123.565367 83.642511) (xy 123.823885 83.31583) (xy 124.088038 82.949593) (xy 124.363409 82.544864)
   (xy 124.970134 81.624181) (xy 125.688719 80.562287) (xy 126.554392 79.373648) (xy 127.0422 78.743392) (xy 127.56467 78.09655)
   (xy 128.120315 77.43865) (xy 128.707646 76.775221) (xy 129.325175 76.111793) (xy 129.971414 75.453893) (xy 130.644873 74.807052)
   (xy 131.344066 74.176797) (xy 132.067503 73.568658) (xy 132.813697 72.988163) (xy 133.581158 72.440842) (xy 134.368399 71.932222)
   (xy 135.173931 71.467834) (xy 135.996266 71.053205) (xy 136.833697 70.692638) (xy 137.683672 70.385503) (xy 138.543427 70.12994)
   (xy 139.410199 69.924087) (xy 140.281222 69.766083) (xy 141.153733 69.654069) (xy 142.024967 69.586182) (xy 142.892161 69.560562))
  (stroke (width 0.105833) (type solid)) (fill no) (layer "Edge.Cuts"))
 (segment (start 95 96) (end 105.794095 85.205905) (width 0.8) (layer "F.Cu") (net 2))
 (segment (start 114.959999 123.999998) (end 110.460001 119.5) (width 0.8) (layer "F.Cu") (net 2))
 (segment (start 113.376276 91.5) (end 115.670371 89.205905) (width 0.8) (layer "F.Cu") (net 2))
 (segment (start 120.305001 104.81) (end 119.69 104.81) (width 0.8) (layer "F.Cu") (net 2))
 (segment (start 120.305001 104.81) (end 123.995001 108.5) (width 0.8) (layer "F.Cu") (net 2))
 (segment (start 121.5 116.5) (end 114.959999 123.040001) (width 0.8) (layer "F.Cu") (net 2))
 (segment (start 123.995001 108.5) (end 130.5 108.5) (width 0.8) (layer "F.Cu") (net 2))
 (segment (start 95 106.5) (end 95 96) (width 0.8) (layer "F.Cu") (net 2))
 (segment (start 120.305001 108.805001) (end 121.5 110) (width 0.8) (layer "F.Cu") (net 2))
 (segment (start 114.959999 123.040001) (end 114.959999 123.999998) (width 0.8) (layer "F.Cu") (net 2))
 (segment (start 111.670371 85.205905) (end 115.670371 89.205905) (width 0.8) (layer "F.Cu") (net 2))
 (segment (start 130.5 103) (end 141.5 92) (width 0.8) (layer "F.Cu") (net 2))
 (segment (start 105.794095 85.205905) (end 111.670371 85.205905) (width 0.8) (layer "F.Cu") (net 2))
 (segment (start 121.5 110) (end 121.5 116.5) (width 0.8) (layer "F.Cu") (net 2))
 (segment (start 130.5 108.5) (end 130.5 103) (width 0.8) (layer "F.Cu") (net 2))
 (segment (start 110.5 91.5) (end 113.376276 91.5) (width 0.8) (layer "F.Cu") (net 2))
 (segment (start 110.460001 119.5) (end 108 119.5) (width 0.8) (layer "F.Cu") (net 2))
 (segment (start 120.305001 104.81) (end 120.305001 108.805001) (width 0.8) (layer "F.Cu") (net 2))
 (segment (start 108 119.5) (end 95 106.5) (width 0.8) (layer "F.Cu") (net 2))
 (segment (start 110 112) (end 112.685001 109.314999) (width 0.8) (layer "F.Cu") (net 3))
 (segment (start 127 96) (end 121.495001 96) (width 0.8) (layer "F.Cu") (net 3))
 (segment (start 120.305001 97.19) (end 112.685001 104.81) (width 0.8) (layer "F.Cu") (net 3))
 (segment (start 135.460442 79.539558) (end 127 88) (width 0.8) (layer "F.Cu") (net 3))
 (segment (start 127 88) (end 127 96) (width 0.8) (layer "F.Cu") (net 3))
 (segment (start 144.838764 79.539558) (end 135.460442 79.539558) (width 0.8) (layer "F.Cu") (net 3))
 (segment (start 112.685001 109.314999) (end 112.685001 104.81) (width 0.8) (layer "F.Cu") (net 3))
 (segment (start 121.495001 96) (end 120.305001 97.19) (width 0.8) (layer "F.Cu") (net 3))
 (segment (start 112.684999 99.73) (end 107.23 99.73) (width 0.8) (layer "F.Cu") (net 5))
 (segment (start 105.670371 90.205905) (end 105.670371 91.209629) (width 0.8) (layer "F.Cu") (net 5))
 (segment (start 105.670371 98.170371) (end 105.670371 90.205905) (width 0.8) (layer "F.Cu") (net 5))
 (segment (start 111.5 116) (end 108 116) (width 0.8) (layer "F.Cu") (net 5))
 (segment (start 115.5 112) (end 111.5 116) (width 0.8) (layer "F.Cu") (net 5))
 (segment (start 120.304998 102.269998) (end 118.730002 102.269998) (width 0.8) (layer "F.Cu") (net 5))
 (segment (start 105.670371 91.209629) (end 102 94.88) (width 0.8) (layer "F.Cu") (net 5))
 (segment (start 98 106) (end 98 98.88) (width 0.8) (layer "F.Cu") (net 5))
 (segment (start 118.730002 102.269998) (end 115.5 105.5) (width 0.8) (layer "F.Cu") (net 5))
 (segment (start 98 98.88) (end 102 94.88) (width 0.8) (layer "F.Cu") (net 5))
 (segment (start 115.5 105.5) (end 115.5 112) (width 0.8) (layer "F.Cu") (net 5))
 (segment (start 108 116) (end 98 106) (width 0.8) (layer "F.Cu") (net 5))
 (segment (start 107.23 99.73) (end 105.670371 98.170371) (width 0.8) (layer "F.Cu") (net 5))
 (segment (start 112.685001 97.19) (end 119.375001 90.5) (width 0.8) (layer "F.Cu") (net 1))
 (segment (start 119.375001 90.5) (end 120.5 90.5) (width 0.8) (layer "F.Cu") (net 1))
 (segment (start 124.19 112.099114) (end 124.19 117.31) (width 0.8) (layer "F.Cu") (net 6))
 (segment (start 124.19 117.31) (end 117.5 124) (width 0.8) (layer "F.Cu") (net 6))
 (segment (start 102 106) (end 102 102.5) (width 0.8) (layer "F.Cu") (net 4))
 (segment (start 108.953691 102.270001) (end 112.685001 102.270001) (width 0.8) (layer "F.Cu") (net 4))
 (segment (start 104.611846 106.611846) (end 108.953691 102.270001) (width 0.8) (layer "F.Cu") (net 4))
 (segment (start 104.611846 106.611846) (end 102.611846 106.611846) (width 0.8) (layer "F.Cu") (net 4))
 (segment (start 102.611846 106.611846) (end 102 106) (width 0.8) (layer "F.Cu") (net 4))
 (segment (start 123.5 100) (end 123.5 105.5) (width 0.8) (layer "F.Cu") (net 7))
 (segment (start 123.23 99.73) (end 123.5 100) (width 0.8) (layer "F.Cu") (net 7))
 (segment (start 123.5 105.5) (end 128 105.5) (width 0.8) (layer "F.Cu") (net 7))
 (segment (start 120.305001 99.73) (end 123.23 99.73) (width 0.8) (layer "F.Cu") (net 7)))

